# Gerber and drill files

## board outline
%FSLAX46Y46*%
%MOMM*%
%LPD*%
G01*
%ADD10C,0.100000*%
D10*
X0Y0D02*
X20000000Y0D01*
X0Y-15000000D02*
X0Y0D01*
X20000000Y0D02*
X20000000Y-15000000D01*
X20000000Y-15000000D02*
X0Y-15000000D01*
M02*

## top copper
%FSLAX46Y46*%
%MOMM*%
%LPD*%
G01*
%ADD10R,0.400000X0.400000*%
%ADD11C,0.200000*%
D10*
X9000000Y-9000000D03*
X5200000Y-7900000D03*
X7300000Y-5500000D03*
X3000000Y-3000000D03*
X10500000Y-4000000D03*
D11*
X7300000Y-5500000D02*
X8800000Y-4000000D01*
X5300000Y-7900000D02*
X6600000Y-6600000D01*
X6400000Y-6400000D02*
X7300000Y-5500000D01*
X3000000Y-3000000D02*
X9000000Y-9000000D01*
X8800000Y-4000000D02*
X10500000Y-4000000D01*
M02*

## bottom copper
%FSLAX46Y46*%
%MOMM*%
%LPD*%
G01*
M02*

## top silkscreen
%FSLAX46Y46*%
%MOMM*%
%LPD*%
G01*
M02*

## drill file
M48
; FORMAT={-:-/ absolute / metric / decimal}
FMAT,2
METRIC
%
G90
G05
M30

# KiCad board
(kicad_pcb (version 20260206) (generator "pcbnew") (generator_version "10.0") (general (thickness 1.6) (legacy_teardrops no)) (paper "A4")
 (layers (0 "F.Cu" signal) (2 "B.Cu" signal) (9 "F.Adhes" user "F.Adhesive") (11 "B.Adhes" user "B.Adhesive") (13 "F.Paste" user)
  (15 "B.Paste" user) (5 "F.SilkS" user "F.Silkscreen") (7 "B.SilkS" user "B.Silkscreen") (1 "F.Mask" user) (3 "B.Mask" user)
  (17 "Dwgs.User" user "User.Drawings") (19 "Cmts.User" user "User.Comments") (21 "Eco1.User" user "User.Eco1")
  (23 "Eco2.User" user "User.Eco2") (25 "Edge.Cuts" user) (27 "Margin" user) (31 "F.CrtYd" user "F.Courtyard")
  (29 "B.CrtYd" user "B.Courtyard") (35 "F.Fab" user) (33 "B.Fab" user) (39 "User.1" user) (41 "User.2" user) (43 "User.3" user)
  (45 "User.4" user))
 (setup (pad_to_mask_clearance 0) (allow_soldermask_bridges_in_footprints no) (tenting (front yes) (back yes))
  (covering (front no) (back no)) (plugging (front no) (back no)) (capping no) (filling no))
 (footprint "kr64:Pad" (layer "F.Cu") (at 9 9)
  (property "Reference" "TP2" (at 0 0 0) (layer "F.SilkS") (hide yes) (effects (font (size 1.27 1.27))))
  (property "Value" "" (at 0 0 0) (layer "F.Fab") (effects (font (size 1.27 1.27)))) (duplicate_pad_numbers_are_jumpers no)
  (pad "1" smd rect (at 0 0) (size 0.4 0.4) (layers "F.Cu" "F.Mask" "F.Paste") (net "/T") (thermal_bridge_angle 45)))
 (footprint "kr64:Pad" (layer "F.Cu") (at 5.2 7.9)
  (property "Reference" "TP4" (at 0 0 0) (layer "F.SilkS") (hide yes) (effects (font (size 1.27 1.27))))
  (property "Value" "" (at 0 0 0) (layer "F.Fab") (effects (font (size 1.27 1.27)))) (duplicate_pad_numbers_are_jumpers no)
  (pad "1" smd rect (at 0 0) (size 0.4 0.4) (layers "F.Cu" "F.Mask" "F.Paste") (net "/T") (thermal_bridge_angle 45)))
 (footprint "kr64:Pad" (layer "F.Cu") (at 7.3 5.5)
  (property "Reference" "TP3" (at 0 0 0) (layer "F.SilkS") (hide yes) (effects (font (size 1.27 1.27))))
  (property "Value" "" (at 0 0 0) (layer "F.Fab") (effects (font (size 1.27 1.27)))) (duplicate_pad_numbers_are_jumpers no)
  (pad "1" smd rect (at 0 0) (size 0.4 0.4) (layers "F.Cu" "F.Mask" "F.Paste") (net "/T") (thermal_bridge_angle 45)))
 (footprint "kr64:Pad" (layer "F.Cu") (at 3 3)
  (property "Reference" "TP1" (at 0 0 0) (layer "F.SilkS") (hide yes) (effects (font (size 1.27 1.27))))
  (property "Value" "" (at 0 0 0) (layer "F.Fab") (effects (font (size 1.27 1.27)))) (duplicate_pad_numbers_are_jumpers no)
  (pad "1" smd rect (at 0 0) (size 0.4 0.4) (layers "F.Cu" "F.Mask" "F.Paste") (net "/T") (thermal_bridge_angle 45)))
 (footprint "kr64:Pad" (layer "F.Cu") (at 10.5 4)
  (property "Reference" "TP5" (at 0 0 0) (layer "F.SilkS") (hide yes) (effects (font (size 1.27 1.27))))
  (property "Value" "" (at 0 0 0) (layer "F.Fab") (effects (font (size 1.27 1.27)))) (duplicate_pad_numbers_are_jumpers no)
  (pad "1" smd rect (at 0 0) (size 0.4 0.4) (layers "F.Cu" "F.Mask" "F.Paste") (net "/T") (thermal_bridge_angle 45)))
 (gr_line (start 0 0) (end 20 0) (stroke (width 0.1) (type default)) (layer "Edge.Cuts"))
 (gr_line (start 0 15) (end 0 0) (stroke (width 0.1) (type default)) (layer "Edge.Cuts"))
 (gr_line (start 20 0) (end 20 15) (stroke (width 0.1) (type default)) (layer "Edge.Cuts"))
 (gr_line (start 20 15) (end 0 15) (stroke (width 0.1) (type default)) (layer "Edge.Cuts"))
 (segment (start 7.3 5.5) (end 8.8 4) (width 0.2) (layer "F.Cu") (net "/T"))
 (segment (start 5.3 7.9) (end 6.6 6.6) (width 0.2) (layer "F.Cu") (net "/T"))
 (segment (start 6.4 6.4) (end 7.3 5.5) (width 0.2) (layer "F.Cu") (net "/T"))
 (segment (start 3 3) (end 9 9) (width 0.2) (layer "F.Cu") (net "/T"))
 (segment (start 8.8 4) (end 10.5 4) (width 0.2) (layer "F.Cu") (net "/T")))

